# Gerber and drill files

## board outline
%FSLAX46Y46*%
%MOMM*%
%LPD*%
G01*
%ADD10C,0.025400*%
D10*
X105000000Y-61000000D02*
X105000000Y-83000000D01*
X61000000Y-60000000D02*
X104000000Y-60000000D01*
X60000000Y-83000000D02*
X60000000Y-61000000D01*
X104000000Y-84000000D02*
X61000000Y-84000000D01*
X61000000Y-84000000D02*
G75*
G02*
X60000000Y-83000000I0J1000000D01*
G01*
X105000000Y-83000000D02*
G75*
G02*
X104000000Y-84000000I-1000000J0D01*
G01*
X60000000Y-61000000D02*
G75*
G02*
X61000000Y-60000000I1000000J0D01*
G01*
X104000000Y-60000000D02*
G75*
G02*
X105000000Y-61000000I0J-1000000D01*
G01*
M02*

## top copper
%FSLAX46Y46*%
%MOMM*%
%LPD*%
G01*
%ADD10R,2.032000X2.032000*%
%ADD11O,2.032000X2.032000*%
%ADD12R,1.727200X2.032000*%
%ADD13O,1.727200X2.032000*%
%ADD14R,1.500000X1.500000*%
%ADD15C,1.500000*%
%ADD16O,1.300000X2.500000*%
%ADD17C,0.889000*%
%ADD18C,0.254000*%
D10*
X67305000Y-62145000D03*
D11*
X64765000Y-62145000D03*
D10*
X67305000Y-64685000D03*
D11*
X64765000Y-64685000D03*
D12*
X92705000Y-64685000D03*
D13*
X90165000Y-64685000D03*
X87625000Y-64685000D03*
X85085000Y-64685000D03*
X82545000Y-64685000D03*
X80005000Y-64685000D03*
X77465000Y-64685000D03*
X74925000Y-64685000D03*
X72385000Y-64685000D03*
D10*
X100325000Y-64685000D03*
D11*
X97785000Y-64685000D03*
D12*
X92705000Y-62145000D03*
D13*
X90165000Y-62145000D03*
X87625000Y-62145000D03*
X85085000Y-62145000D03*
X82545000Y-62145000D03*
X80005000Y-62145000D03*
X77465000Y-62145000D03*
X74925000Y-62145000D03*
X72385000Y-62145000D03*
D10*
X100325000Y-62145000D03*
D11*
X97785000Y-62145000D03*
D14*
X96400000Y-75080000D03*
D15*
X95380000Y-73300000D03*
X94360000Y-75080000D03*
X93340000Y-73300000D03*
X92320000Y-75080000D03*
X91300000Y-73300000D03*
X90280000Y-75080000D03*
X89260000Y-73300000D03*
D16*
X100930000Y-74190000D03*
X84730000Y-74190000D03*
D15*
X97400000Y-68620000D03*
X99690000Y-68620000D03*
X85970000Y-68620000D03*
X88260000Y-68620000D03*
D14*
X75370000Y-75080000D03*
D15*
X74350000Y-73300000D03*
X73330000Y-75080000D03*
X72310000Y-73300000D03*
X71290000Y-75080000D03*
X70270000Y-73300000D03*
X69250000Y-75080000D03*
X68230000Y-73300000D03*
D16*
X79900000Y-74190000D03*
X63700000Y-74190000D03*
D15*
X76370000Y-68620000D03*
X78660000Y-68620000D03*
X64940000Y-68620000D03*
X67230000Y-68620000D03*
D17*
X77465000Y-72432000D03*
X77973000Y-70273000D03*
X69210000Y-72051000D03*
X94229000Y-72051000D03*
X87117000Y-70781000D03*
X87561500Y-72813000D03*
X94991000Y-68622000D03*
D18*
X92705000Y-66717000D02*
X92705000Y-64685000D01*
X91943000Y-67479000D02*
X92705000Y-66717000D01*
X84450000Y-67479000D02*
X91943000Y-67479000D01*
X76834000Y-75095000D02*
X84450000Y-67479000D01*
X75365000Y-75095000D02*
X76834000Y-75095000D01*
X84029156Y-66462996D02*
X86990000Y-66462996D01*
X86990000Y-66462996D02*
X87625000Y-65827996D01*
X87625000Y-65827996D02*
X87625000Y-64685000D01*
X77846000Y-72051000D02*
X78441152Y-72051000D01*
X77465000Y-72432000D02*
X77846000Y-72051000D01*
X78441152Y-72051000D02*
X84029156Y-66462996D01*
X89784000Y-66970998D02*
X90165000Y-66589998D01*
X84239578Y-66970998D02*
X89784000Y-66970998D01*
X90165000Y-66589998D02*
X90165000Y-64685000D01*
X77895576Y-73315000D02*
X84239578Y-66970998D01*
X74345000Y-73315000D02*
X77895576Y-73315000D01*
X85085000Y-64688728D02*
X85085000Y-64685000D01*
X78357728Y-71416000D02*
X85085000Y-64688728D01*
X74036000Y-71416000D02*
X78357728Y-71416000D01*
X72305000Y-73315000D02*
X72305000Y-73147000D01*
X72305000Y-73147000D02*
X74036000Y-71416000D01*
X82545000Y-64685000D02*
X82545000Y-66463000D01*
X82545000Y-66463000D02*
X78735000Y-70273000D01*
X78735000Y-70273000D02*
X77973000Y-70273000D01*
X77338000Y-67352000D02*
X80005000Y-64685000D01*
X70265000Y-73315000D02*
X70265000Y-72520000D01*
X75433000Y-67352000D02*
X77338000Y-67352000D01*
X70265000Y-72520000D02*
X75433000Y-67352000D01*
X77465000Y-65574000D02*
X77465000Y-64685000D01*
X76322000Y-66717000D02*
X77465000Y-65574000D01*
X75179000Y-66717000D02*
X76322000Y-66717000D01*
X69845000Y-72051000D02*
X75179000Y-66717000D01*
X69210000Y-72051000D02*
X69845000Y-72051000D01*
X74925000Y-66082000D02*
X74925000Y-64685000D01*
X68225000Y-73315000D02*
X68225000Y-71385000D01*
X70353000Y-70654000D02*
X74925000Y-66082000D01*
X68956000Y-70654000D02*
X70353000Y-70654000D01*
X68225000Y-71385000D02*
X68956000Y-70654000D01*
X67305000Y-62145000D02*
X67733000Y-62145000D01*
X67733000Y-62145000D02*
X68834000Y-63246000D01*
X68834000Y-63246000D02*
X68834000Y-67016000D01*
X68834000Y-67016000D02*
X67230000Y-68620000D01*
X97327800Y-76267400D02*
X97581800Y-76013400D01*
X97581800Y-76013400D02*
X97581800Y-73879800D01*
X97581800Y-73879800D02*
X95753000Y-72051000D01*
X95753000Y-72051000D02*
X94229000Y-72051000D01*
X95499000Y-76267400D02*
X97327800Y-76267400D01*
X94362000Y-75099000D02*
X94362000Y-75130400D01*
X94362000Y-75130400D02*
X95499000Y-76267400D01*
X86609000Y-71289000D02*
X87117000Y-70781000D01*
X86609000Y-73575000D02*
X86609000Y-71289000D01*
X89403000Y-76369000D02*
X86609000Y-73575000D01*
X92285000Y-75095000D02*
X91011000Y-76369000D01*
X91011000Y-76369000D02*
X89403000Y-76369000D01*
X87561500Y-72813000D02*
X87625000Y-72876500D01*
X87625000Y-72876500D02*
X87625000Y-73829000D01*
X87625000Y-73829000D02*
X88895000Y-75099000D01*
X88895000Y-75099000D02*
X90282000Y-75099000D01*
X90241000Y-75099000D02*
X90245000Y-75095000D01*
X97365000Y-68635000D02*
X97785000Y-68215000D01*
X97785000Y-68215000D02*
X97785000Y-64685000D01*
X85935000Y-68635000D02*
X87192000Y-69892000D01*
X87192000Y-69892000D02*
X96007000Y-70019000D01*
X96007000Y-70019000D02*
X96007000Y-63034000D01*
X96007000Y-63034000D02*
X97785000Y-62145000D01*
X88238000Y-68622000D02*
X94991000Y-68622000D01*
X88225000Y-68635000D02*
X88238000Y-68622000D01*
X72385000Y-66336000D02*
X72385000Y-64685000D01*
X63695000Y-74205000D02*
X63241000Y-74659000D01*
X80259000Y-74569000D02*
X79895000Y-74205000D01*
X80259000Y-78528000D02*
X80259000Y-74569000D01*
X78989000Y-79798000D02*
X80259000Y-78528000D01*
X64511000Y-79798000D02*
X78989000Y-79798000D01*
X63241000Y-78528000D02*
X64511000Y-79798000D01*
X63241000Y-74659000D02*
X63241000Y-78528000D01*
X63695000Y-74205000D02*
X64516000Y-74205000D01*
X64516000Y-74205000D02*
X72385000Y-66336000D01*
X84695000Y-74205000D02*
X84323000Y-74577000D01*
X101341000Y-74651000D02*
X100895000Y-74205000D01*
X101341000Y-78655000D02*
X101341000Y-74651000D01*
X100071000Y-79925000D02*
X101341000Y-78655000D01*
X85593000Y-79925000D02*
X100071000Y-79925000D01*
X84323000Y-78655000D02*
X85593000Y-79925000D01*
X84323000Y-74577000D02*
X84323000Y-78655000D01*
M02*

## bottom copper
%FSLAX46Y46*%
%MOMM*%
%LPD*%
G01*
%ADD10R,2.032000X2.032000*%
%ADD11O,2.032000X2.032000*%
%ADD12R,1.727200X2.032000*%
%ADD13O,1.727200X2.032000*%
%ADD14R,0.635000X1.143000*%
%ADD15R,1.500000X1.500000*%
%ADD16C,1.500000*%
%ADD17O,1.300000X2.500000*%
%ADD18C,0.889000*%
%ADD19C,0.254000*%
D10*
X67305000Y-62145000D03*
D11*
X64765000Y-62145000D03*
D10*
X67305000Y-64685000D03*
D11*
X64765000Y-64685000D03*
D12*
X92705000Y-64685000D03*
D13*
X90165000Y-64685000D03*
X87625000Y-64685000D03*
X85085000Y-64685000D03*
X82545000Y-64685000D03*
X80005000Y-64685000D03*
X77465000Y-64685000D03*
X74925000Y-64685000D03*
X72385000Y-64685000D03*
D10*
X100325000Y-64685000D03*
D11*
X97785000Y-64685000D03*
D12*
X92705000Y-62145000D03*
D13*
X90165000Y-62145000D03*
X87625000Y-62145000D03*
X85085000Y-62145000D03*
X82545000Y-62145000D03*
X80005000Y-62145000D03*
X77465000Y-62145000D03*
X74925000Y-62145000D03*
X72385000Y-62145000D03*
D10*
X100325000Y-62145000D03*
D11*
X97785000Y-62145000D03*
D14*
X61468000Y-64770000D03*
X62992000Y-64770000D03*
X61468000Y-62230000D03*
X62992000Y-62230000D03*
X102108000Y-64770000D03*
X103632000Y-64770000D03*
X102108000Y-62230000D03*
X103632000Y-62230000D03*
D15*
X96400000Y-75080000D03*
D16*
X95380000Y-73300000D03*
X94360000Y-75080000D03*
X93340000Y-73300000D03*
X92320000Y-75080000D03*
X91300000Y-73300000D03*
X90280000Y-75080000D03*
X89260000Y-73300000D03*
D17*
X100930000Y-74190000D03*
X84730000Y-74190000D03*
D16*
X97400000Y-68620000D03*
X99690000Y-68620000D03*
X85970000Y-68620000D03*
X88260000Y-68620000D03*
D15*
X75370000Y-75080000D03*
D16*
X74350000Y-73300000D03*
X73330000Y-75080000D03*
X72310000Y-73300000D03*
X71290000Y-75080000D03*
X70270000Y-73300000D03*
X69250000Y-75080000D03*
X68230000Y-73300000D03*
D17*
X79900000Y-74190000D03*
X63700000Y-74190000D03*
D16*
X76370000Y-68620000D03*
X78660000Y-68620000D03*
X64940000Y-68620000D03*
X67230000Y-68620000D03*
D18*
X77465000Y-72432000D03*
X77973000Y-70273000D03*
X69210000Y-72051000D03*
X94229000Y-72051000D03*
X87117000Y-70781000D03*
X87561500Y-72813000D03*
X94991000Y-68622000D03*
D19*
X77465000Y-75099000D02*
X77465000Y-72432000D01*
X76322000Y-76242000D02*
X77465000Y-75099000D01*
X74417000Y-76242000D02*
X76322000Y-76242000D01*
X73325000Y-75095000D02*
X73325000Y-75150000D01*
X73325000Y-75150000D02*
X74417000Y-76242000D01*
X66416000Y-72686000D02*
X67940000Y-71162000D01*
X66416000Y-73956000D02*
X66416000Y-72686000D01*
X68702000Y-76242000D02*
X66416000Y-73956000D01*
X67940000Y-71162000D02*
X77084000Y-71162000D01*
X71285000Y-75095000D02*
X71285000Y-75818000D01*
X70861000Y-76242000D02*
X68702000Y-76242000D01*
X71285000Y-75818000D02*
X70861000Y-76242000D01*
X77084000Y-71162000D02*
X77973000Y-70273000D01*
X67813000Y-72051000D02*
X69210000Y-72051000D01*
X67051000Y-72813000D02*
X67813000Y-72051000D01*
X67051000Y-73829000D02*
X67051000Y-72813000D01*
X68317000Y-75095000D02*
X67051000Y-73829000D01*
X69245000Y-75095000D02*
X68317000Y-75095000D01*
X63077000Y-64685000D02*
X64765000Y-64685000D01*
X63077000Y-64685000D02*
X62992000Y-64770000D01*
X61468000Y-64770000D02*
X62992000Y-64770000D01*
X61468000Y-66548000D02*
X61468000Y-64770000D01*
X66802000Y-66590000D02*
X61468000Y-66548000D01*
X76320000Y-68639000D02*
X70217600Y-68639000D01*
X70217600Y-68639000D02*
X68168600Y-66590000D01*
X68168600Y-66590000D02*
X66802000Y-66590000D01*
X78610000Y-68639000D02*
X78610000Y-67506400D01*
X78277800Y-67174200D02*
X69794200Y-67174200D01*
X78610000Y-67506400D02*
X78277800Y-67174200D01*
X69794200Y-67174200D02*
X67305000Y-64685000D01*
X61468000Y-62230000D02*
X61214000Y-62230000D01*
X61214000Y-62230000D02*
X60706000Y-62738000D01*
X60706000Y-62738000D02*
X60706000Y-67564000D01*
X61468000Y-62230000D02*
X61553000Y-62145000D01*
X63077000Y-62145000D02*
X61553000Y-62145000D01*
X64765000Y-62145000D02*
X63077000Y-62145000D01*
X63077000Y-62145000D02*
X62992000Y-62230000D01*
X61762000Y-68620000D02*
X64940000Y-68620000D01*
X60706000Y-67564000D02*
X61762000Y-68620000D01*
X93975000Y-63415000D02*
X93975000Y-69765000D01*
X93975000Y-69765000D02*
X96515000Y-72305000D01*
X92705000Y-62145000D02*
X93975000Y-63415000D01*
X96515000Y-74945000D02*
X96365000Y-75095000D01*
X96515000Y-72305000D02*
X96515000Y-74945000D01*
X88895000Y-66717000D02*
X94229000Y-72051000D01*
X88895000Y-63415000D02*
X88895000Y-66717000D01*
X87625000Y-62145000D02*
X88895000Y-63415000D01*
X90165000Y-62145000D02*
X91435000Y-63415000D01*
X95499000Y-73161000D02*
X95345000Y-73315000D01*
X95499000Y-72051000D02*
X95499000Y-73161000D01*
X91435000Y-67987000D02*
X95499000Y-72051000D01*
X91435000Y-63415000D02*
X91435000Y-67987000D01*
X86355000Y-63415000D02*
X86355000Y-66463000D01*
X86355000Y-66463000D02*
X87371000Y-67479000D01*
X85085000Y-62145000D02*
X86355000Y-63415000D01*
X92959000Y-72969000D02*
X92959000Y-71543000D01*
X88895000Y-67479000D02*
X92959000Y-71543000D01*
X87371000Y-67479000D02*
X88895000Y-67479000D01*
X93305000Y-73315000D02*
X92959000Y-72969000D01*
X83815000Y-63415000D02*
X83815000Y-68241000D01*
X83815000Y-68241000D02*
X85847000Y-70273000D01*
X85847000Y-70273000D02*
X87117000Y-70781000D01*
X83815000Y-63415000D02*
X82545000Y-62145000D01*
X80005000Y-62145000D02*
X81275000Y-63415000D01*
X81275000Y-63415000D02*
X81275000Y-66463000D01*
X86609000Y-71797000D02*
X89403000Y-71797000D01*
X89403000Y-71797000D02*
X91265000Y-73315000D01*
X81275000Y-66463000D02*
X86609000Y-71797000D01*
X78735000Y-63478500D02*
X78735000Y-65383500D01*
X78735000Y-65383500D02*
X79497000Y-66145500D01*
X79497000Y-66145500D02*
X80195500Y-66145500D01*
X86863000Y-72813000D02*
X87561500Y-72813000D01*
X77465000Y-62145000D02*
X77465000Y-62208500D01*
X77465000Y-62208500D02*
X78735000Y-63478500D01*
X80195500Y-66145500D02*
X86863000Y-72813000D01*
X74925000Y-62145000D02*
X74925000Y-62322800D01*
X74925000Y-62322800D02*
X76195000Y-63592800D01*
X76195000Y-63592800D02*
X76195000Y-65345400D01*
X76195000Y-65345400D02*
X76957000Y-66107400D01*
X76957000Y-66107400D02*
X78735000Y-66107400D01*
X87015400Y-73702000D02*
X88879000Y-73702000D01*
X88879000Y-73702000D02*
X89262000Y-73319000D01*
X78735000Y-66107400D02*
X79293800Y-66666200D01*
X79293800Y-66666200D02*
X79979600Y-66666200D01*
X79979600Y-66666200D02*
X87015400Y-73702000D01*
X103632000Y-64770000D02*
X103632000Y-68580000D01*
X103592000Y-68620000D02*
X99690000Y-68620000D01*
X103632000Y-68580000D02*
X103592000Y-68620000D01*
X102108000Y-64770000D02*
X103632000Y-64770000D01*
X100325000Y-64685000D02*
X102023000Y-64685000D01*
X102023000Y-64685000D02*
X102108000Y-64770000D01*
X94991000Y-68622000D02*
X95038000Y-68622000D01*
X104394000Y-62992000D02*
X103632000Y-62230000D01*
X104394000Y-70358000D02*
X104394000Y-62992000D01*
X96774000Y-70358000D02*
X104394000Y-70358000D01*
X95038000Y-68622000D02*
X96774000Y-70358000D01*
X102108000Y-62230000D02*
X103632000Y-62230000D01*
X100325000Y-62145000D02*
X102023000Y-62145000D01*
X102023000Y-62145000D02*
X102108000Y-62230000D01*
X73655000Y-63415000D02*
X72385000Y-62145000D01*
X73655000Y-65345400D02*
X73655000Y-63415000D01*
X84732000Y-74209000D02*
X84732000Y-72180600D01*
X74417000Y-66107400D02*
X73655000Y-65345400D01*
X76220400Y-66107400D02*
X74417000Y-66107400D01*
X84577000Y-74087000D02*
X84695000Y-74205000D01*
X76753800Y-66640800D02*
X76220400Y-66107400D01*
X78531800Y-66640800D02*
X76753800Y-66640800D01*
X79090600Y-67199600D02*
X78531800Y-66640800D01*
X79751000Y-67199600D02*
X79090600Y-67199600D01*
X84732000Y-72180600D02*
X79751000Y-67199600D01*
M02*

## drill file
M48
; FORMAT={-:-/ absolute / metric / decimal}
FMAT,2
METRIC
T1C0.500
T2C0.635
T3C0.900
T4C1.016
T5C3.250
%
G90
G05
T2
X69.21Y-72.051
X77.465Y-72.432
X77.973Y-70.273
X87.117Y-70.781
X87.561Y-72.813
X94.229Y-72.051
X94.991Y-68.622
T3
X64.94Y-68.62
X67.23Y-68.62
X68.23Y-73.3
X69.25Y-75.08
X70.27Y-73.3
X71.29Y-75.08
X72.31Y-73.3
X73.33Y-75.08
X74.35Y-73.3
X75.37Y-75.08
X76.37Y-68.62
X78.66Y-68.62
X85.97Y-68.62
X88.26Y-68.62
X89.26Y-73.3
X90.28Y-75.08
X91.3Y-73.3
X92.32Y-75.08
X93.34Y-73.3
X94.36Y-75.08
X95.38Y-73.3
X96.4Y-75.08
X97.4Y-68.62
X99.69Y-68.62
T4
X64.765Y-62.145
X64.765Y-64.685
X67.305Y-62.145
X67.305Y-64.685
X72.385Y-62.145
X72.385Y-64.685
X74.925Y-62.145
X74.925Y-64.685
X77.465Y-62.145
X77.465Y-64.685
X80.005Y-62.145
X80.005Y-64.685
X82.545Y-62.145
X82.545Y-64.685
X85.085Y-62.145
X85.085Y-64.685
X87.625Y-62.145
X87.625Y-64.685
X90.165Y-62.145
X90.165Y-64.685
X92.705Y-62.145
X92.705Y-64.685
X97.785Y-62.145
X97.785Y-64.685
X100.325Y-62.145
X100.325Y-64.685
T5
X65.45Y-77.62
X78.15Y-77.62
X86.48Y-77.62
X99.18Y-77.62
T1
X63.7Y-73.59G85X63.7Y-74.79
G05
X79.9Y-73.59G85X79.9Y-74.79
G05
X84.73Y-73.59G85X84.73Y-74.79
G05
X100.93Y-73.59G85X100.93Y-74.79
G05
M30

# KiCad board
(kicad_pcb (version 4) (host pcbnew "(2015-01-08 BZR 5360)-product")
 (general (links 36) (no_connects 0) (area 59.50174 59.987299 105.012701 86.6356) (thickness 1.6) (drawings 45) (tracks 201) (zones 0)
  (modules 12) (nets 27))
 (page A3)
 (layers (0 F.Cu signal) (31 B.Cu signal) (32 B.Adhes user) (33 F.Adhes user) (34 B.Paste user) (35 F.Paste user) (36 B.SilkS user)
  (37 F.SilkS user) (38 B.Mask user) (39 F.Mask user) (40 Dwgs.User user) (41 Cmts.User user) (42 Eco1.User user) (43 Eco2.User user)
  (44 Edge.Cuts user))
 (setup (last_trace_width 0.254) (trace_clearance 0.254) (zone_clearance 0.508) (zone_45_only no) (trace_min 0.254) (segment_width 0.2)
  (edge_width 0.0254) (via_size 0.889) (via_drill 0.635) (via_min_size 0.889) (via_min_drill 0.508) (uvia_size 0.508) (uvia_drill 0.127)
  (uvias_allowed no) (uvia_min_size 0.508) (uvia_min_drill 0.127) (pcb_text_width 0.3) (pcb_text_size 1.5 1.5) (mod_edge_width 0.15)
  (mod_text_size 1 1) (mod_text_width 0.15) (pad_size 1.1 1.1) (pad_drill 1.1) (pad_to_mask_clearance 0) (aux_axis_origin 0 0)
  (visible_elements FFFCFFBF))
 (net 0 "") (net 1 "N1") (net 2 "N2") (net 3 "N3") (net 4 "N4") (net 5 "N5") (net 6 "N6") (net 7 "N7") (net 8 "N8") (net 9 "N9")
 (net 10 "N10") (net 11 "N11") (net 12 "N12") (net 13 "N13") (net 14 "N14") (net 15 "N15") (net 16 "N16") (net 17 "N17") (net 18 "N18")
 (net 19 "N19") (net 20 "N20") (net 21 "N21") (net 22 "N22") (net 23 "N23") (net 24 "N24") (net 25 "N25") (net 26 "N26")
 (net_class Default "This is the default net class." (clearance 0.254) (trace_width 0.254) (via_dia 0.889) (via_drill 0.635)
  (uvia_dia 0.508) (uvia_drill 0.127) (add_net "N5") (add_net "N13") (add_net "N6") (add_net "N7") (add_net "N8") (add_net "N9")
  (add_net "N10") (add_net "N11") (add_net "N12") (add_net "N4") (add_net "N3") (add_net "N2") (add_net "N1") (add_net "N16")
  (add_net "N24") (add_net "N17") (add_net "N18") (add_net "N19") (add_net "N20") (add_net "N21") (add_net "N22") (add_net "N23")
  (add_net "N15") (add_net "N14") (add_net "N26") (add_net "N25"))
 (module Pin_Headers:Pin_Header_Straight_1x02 (layer F.Cu) (at 66.035 62.145 180)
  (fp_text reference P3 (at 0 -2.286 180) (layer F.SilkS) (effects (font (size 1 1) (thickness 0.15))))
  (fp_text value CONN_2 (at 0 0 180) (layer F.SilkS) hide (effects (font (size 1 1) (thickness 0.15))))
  (pad 1 thru_hole rect (at -1.27 0 180) (size 2.032 2.032) (drill 1.016) (layers *.Cu *.Mask F.SilkS) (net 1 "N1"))
  (pad 2 thru_hole oval (at 1.27 0 180) (size 2.032 2.032) (drill 1.016) (layers *.Cu *.Mask F.SilkS) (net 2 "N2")))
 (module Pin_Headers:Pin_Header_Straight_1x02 (layer F.Cu) (at 66.035 64.685 180)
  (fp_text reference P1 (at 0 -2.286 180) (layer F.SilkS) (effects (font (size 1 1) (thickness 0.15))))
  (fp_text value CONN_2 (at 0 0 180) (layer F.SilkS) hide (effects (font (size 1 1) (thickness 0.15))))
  (pad 1 thru_hole rect (at -1.27 0 180) (size 2.032 2.032) (drill 1.016) (layers *.Cu *.Mask F.SilkS) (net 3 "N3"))
  (pad 2 thru_hole oval (at 1.27 0 180) (size 2.032 2.032) (drill 1.016) (layers *.Cu *.Mask F.SilkS) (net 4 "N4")))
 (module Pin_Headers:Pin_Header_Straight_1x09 (layer F.Cu) (at 82.545 64.685 180)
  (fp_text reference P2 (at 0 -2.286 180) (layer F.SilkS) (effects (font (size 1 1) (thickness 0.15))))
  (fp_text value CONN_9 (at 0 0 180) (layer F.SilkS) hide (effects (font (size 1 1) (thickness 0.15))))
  (pad 1 thru_hole rect (at -10.16 0 180) (size 1.7272 2.032) (drill 1.016) (layers *.Cu *.Mask F.SilkS) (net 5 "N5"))
  (pad 2 thru_hole oval (at -7.62 0 180) (size 1.7272 2.032) (drill 1.016) (layers *.Cu *.Mask F.SilkS) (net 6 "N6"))
  (pad 3 thru_hole oval (at -5.08 0 180) (size 1.7272 2.032) (drill 1.016) (layers *.Cu *.Mask F.SilkS) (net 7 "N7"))
  (pad 4 thru_hole oval (at -2.54 0 180) (size 1.7272 2.032) (drill 1.016) (layers *.Cu *.Mask F.SilkS) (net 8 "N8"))
  (pad 5 thru_hole oval (at 0 0 180) (size 1.7272 2.032) (drill 1.016) (layers *.Cu *.Mask F.SilkS) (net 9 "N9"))
  (pad 6 thru_hole oval (at 2.54 0 180) (size 1.7272 2.032) (drill 1.016) (layers *.Cu *.Mask F.SilkS) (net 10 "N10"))
  (pad 7 thru_hole oval (at 5.08 0 180) (size 1.7272 2.032) (drill 1.016) (layers *.Cu *.Mask F.SilkS) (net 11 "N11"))
  (pad 8 thru_hole oval (at 7.62 0 180) (size 1.7272 2.032) (drill 1.016) (layers *.Cu *.Mask F.SilkS) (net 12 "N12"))
  (pad 9 thru_hole oval (at 10.16 0 180) (size 1.7272 2.032) (drill 1.016) (layers *.Cu *.Mask F.SilkS) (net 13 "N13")))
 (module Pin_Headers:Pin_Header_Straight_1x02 (layer F.Cu) (at 99.055 64.685 180)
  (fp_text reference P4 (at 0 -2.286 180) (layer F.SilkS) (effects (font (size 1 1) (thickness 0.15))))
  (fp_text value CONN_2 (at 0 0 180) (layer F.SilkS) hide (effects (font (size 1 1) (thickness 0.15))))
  (pad 1 thru_hole rect (at -1.27 0 180) (size 2.032 2.032) (drill 1.016) (layers *.Cu *.Mask F.SilkS) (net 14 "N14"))
  (pad 2 thru_hole oval (at 1.27 0 180) (size 2.032 2.032) (drill 1.016) (layers *.Cu *.Mask F.SilkS) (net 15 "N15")))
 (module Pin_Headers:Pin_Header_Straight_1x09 (layer F.Cu) (at 82.545 62.145 180)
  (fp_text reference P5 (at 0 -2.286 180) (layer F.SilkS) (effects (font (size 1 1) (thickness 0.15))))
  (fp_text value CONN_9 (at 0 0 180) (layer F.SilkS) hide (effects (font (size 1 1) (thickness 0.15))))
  (pad 1 thru_hole rect (at -10.16 0 180) (size 1.7272 2.032) (drill 1.016) (layers *.Cu *.Mask F.SilkS) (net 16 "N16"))
  (pad 2 thru_hole oval (at -7.62 0 180) (size 1.7272 2.032) (drill 1.016) (layers *.Cu *.Mask F.SilkS) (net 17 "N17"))
  (pad 3 thru_hole oval (at -5.08 0 180) (size 1.7272 2.032) (drill 1.016) (layers *.Cu *.Mask F.SilkS) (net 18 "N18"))
  (pad 4 thru_hole oval (at -2.54 0 180) (size 1.7272 2.032) (drill 1.016) (layers *.Cu *.Mask F.SilkS) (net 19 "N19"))
  (pad 5 thru_hole oval (at 0 0 180) (size 1.7272 2.032) (drill 1.016) (layers *.Cu *.Mask F.SilkS) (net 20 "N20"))
  (pad 6 thru_hole oval (at 2.54 0 180) (size 1.7272 2.032) (drill 1.016) (layers *.Cu *.Mask F.SilkS) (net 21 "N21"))
  (pad 7 thru_hole oval (at 5.08 0 180) (size 1.7272 2.032) (drill 1.016) (layers *.Cu *.Mask F.SilkS) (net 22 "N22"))
  (pad 8 thru_hole oval (at 7.62 0 180) (size 1.7272 2.032) (drill 1.016) (layers *.Cu *.Mask F.SilkS) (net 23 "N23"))
  (pad 9 thru_hole oval (at 10.16 0 180) (size 1.7272 2.032) (drill 1.016) (layers *.Cu *.Mask F.SilkS) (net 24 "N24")))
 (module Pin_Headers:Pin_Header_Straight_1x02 (layer F.Cu) (at 99.055 62.145 180)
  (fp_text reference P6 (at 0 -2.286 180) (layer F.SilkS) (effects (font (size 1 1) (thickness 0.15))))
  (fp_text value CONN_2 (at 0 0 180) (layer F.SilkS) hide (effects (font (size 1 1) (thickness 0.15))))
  (pad 1 thru_hole rect (at -1.27 0 180) (size 2.032 2.032) (drill 1.016) (layers *.Cu *.Mask F.SilkS) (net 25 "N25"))
  (pad 2 thru_hole oval (at 1.27 0 180) (size 2.032 2.032) (drill 1.016) (layers *.Cu *.Mask F.SilkS) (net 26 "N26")))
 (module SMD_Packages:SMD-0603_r (layer B.Cu) (at 62.23 64.77)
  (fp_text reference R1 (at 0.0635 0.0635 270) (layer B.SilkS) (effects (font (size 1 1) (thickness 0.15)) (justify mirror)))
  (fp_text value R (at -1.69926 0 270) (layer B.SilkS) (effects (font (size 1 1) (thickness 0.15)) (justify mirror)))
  (pad 1 smd rect (at -0.762 0) (size 0.635 1.143) (layers B.Cu B.Paste B.Mask) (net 4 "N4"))
  (pad 2 smd rect (at 0.762 0) (size 0.635 1.143) (layers B.Cu B.Paste B.Mask) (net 4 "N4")))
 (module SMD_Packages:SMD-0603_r (layer B.Cu) (at 62.23 62.23)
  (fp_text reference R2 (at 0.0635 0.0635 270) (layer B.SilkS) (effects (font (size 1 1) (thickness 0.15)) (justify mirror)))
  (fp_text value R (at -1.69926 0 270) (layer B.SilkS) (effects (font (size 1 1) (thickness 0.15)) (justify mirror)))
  (pad 1 smd rect (at -0.762 0) (size 0.635 1.143) (layers B.Cu B.Paste B.Mask) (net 2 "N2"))
  (pad 2 smd rect (at 0.762 0) (size 0.635 1.143) (layers B.Cu B.Paste B.Mask) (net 2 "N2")))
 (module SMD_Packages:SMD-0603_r (layer B.Cu) (at 102.87 64.77)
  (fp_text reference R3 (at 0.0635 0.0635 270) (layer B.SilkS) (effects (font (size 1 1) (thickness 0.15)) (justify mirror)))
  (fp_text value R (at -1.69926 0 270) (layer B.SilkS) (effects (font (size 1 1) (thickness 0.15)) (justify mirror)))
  (pad 1 smd rect (at -0.762 0) (size 0.635 1.143) (layers B.Cu B.Paste B.Mask) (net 14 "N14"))
  (pad 2 smd rect (at 0.762 0) (size 0.635 1.143) (layers B.Cu B.Paste B.Mask) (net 14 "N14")))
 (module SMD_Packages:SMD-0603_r (layer B.Cu) (at 102.87 62.23)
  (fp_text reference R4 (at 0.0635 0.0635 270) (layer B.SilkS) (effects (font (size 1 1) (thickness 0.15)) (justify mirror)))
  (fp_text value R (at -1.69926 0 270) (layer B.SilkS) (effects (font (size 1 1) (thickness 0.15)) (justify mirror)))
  (pad 1 smd rect (at -0.762 0) (size 0.635 1.143) (layers B.Cu B.Paste B.Mask) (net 25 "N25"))
  (pad 2 smd rect (at 0.762 0) (size 0.635 1.143) (layers B.Cu B.Paste B.Mask) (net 25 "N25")))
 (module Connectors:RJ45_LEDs (layer F.Cu) (at 96.4 75.08 180)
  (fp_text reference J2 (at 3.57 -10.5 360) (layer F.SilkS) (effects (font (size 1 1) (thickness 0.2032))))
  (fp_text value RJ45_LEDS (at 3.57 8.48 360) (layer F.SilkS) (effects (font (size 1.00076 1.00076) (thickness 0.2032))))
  (pad 1 thru_hole rect (at 0 0) (size 1.5 1.5) (drill 0.9) (layers *.Cu *.Mask F.SilkS) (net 16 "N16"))
  (pad 2 thru_hole circle (at 1.02 1.78) (size 1.5 1.5) (drill 0.9) (layers *.Cu *.Mask F.SilkS) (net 17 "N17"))
  (pad 3 thru_hole circle (at 2.04 0) (size 1.5 1.5) (drill 0.9) (layers *.Cu *.Mask F.SilkS) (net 18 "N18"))
  (pad 4 thru_hole circle (at 3.06 1.78) (size 1.5 1.5) (drill 0.9) (layers *.Cu *.Mask F.SilkS) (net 19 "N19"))
  (pad 5 thru_hole circle (at 4.08 0) (size 1.5 1.5) (drill 0.9) (layers *.Cu *.Mask F.SilkS) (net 20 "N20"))
  (pad 6 thru_hole circle (at 5.1 1.78) (size 1.5 1.5) (drill 0.9) (layers *.Cu *.Mask F.SilkS) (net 21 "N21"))
  (pad 7 thru_hole circle (at 6.12 0) (size 1.5 1.5) (drill 0.9) (layers *.Cu *.Mask F.SilkS) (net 22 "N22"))
  (pad 8 thru_hole circle (at 7.14 1.78) (size 1.5 1.5) (drill 0.9) (layers *.Cu *.Mask F.SilkS) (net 23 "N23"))
  (pad 13 thru_hole oval (at -4.53 0.89) (size 1.3 2.5) (drill oval 0.5 1.7) (layers *.Cu *.Mask F.SilkS) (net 24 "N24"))
  (pad 13 thru_hole oval (at 11.67 0.89) (size 1.3 2.5) (drill oval 0.5 1.7) (layers *.Cu *.Mask F.SilkS) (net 24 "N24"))
  (pad GA thru_hole circle (at -1 6.46) (size 1.5 1.5) (drill 0.9) (layers *.Cu *.Mask F.SilkS) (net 15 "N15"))
  (pad "" np_thru_hole circle (at -2.78 -2.54) (size 3.25 3.25) (drill 3.25) (layers *.Cu *.Mask F.SilkS))
  (pad "" np_thru_hole circle (at 9.92 -2.54) (size 3.25 3.25) (drill 3.25) (layers *.Cu *.Mask F.SilkS))
  (pad GK thru_hole circle (at -3.29 6.46) (size 1.5 1.5) (drill 0.9) (layers *.Cu *.Mask F.SilkS) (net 14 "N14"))
  (pad YA thru_hole circle (at 10.43 6.46) (size 1.5 1.5) (drill 0.9) (layers *.Cu *.Mask F.SilkS) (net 26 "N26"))
  (pad YK thru_hole circle (at 8.14 6.46) (size 1.5 1.5) (drill 0.9) (layers *.Cu *.Mask F.SilkS) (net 25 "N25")))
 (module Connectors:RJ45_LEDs (layer F.Cu) (at 75.37 75.08 180)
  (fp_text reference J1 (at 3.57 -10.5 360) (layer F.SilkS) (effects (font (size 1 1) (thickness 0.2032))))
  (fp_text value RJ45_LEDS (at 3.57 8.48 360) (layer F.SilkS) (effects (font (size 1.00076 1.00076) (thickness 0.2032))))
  (pad 1 thru_hole rect (at 0 0) (size 1.5 1.5) (drill 0.9) (layers *.Cu *.Mask F.SilkS) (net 5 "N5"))
  (pad 2 thru_hole circle (at 1.02 1.78) (size 1.5 1.5) (drill 0.9) (layers *.Cu *.Mask F.SilkS) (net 6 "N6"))
  (pad 3 thru_hole circle (at 2.04 0) (size 1.5 1.5) (drill 0.9) (layers *.Cu *.Mask F.SilkS) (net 7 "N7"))
  (pad 4 thru_hole circle (at 3.06 1.78) (size 1.5 1.5) (drill 0.9) (layers *.Cu *.Mask F.SilkS) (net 8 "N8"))
  (pad 5 thru_hole circle (at 4.08 0) (size 1.5 1.5) (drill 0.9) (layers *.Cu *.Mask F.SilkS) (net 9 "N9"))
  (pad 6 thru_hole circle (at 5.1 1.78) (size 1.5 1.5) (drill 0.9) (layers *.Cu *.Mask F.SilkS) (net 10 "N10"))
  (pad 7 thru_hole circle (at 6.12 0) (size 1.5 1.5) (drill 0.9) (layers *.Cu *.Mask F.SilkS) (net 11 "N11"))
  (pad 8 thru_hole circle (at 7.14 1.78) (size 1.5 1.5) (drill 0.9) (layers *.Cu *.Mask F.SilkS) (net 12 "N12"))
  (pad 13 thru_hole oval (at -4.53 0.89) (size 1.3 2.5) (drill oval 0.5 1.7) (layers *.Cu *.Mask F.SilkS) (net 13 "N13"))
  (pad 13 thru_hole oval (at 11.67 0.89) (size 1.3 2.5) (drill oval 0.5 1.7) (layers *.Cu *.Mask F.SilkS) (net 13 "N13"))
  (pad GA thru_hole circle (at -1 6.46) (size 1.5 1.5) (drill 0.9) (layers *.Cu *.Mask F.SilkS) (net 4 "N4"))
  (pad "" np_thru_hole circle (at -2.78 -2.54) (size 3.25 3.25) (drill 3.25) (layers *.Cu *.Mask F.SilkS))
  (pad "" np_thru_hole circle (at 9.92 -2.54) (size 3.25 3.25) (drill 3.25) (layers *.Cu *.Mask F.SilkS))
  (pad GK thru_hole circle (at -3.29 6.46) (size 1.5 1.5) (drill 0.9) (layers *.Cu *.Mask F.SilkS) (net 3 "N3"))
  (pad YA thru_hole circle (at 10.43 6.46) (size 1.5 1.5) (drill 0.9) (layers *.Cu *.Mask F.SilkS) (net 2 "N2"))
  (pad YK thru_hole circle (at 8.14 6.46) (size 1.5 1.5) (drill 0.9) (layers *.Cu *.Mask F.SilkS) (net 1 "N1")))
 (gr_line (start 105 61) (end 105 83) (angle 90) (layer Edge.Cuts) (width 0.0254))
 (gr_line (start 61 60) (end 104 60) (angle 90) (layer Edge.Cuts) (width 0.0254))
 (gr_line (start 60 83) (end 60 61) (angle 90) (layer Edge.Cuts) (width 0.0254))
 (gr_line (start 104 84) (end 61 84) (angle 90) (layer Edge.Cuts) (width 0.0254))
 (gr_arc (start 61 83) (end 61 84) (angle 90) (layer Edge.Cuts) (width 0.0254))
 (gr_arc (start 104 83) (end 105 83) (angle 90) (layer Edge.Cuts) (width 0.0254))
 (gr_arc (start 61 61) (end 60 61) (angle 90) (layer Edge.Cuts) (width 0.0254))
 (gr_arc (start 104 61) (end 104 60) (angle 90) (layer Edge.Cuts) (width 0.0254))
 (segment (start 92.705 66.717) (end 92.705 64.685) (width 0.254) (layer F.Cu) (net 5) (status 20))
 (segment (start 91.943 67.479) (end 92.705 66.717) (width 0.254) (layer F.Cu) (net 5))
 (segment (start 84.45 67.479) (end 91.943 67.479) (width 0.254) (layer F.Cu) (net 5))
 (segment (start 76.834 75.095) (end 84.45 67.479) (width 0.254) (layer F.Cu) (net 5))
 (segment (start 75.365 75.095) (end 76.834 75.095) (width 0.254) (layer F.Cu) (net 5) (status 10))
 (segment (start 84.029156 66.462996) (end 86.99 66.462996) (width 0.254) (layer F.Cu) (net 7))
 (segment (start 86.99 66.462996) (end 87.625 65.827996) (width 0.254) (layer F.Cu) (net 7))
 (segment (start 87.625 65.827996) (end 87.625 64.685) (width 0.254) (layer F.Cu) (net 7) (status 20))
 (via (at 77.465 72.432) (size 0.889) (layers F.Cu B.Cu) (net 7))
 (segment (start 77.465 75.099) (end 77.465 72.432) (width 0.254) (layer B.Cu) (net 7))
 (segment (start 76.322 76.242) (end 77.465 75.099) (width 0.254) (layer B.Cu) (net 7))
 (segment (start 77.846 72.051) (end 78.441152 72.051) (width 0.254) (layer F.Cu) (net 7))
 (segment (start 77.465 72.432) (end 77.846 72.051) (width 0.254) (layer F.Cu) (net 7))
 (segment (start 78.441152 72.051) (end 84.029156 66.462996) (width 0.254) (layer F.Cu) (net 7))
 (segment (start 74.417 76.242) (end 76.322 76.242) (width 0.254) (layer B.Cu) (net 7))
 (segment (start 73.325 75.095) (end 73.325 75.15) (width 0.254) (layer B.Cu) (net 7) (status 30))
 (segment (start 73.325 75.15) (end 74.417 76.242) (width 0.254) (layer B.Cu) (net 7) (status 10))
 (segment (start 89.784 66.970998) (end 90.165 66.589998) (width 0.254) (layer F.Cu) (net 6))
 (segment (start 84.239578 66.970998) (end 89.784 66.970998) (width 0.254) (layer F.Cu) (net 6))
 (segment (start 90.165 66.589998) (end 90.165 64.685) (width 0.254) (layer F.Cu) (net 6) (status 20))
 (segment (start 77.895576 73.315) (end 84.239578 66.970998) (width 0.254) (layer F.Cu) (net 6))
 (segment (start 74.345 73.315) (end 77.895576 73.315) (width 0.254) (layer F.Cu) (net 6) (status 10))
 (segment (start 85.085 64.688728) (end 85.085 64.685) (width 0.254) (layer F.Cu) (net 8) (status 30))
 (segment (start 78.357728 71.416) (end 85.085 64.688728) (width 0.254) (layer F.Cu) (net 8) (status 20))
 (segment (start 74.036 71.416) (end 78.357728 71.416) (width 0.254) (layer F.Cu) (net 8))
 (segment (start 72.305 73.315) (end 72.305 73.147) (width 0.254) (layer F.Cu) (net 8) (status 30))
 (segment (start 72.305 73.147) (end 74.036 71.416) (width 0.254) (layer F.Cu) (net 8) (status 10))
 (segment (start 82.545 64.685) (end 82.545 66.463) (width 0.254) (layer F.Cu) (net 9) (status 10))
 (segment (start 66.416 72.686) (end 67.94 71.162) (width 0.254) (layer B.Cu) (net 9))
 (segment (start 66.416 73.956) (end 66.416 72.686) (width 0.254) (layer B.Cu) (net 9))
 (segment (start 68.702 76.242) (end 66.416 73.956) (width 0.254) (layer B.Cu) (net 9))
 (segment (start 67.94 71.162) (end 77.084 71.162) (width 0.254) (layer B.Cu) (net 9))
 (segment (start 71.285 75.095) (end 71.285 75.818) (width 0.254) (layer B.Cu) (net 9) (status 30))
 (segment (start 70.861 76.242) (end 68.702 76.242) (width 0.254) (layer B.Cu) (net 9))
 (segment (start 71.285 75.818) (end 70.861 76.242) (width 0.254) (layer B.Cu) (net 9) (status 10))
 (segment (start 77.084 71.162) (end 77.973 70.273) (width 0.254) (layer B.Cu) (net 9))
 (via (at 77.973 70.273) (size 0.889) (layers F.Cu B.Cu) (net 9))
 (segment (start 82.545 66.463) (end 78.735 70.273) (width 0.254) (layer F.Cu) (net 9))
 (segment (start 78.735 70.273) (end 77.973 70.273) (width 0.254) (layer F.Cu) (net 9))
 (segment (start 77.338 67.352) (end 80.005 64.685) (width 0.254) (layer F.Cu) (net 10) (status 20))
 (segment (start 70.265 73.315) (end 70.265 72.52) (width 0.254) (layer F.Cu) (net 10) (status 10))
 (segment (start 75.433 67.352) (end 77.338 67.352) (width 0.254) (layer F.Cu) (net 10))
 (segment (start 70.265 72.52) (end 75.433 67.352) (width 0.254) (layer F.Cu) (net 10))
 (segment (start 77.465 65.574) (end 77.465 64.685) (width 0.254) (layer F.Cu) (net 11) (status 30))
 (segment (start 76.322 66.717) (end 77.465 65.574) (width 0.254) (layer F.Cu) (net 11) (status 20))
 (segment (start 75.179 66.717) (end 76.322 66.717) (width 0.254) (layer F.Cu) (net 11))
 (segment (start 69.845 72.051) (end 75.179 66.717) (width 0.254) (layer F.Cu) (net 11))
 (segment (start 69.21 72.051) (end 69.845 72.051) (width 0.254) (layer F.Cu) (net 11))
 (via (at 69.21 72.051) (size 0.889) (layers F.Cu B.Cu) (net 11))
 (segment (start 67.813 72.051) (end 69.21 72.051) (width 0.254) (layer B.Cu) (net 11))
 (segment (start 67.051 72.813) (end 67.813 72.051) (width 0.254) (layer B.Cu) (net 11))
 (segment (start 67.051 73.829) (end 67.051 72.813) (width 0.254) (layer B.Cu) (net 11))
 (segment (start 68.317 75.095) (end 67.051 73.829) (width 0.254) (layer B.Cu) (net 11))
 (segment (start 69.245 75.095) (end 68.317 75.095) (width 0.254) (layer B.Cu) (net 11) (status 10))
 (segment (start 74.925 66.082) (end 74.925 64.685) (width 0.254) (layer F.Cu) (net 12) (status 20))
 (segment (start 68.225 73.315) (end 68.225 71.385) (width 0.254) (layer F.Cu) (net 12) (status 10))
 (segment (start 70.353 70.654) (end 74.925 66.082) (width 0.254) (layer F.Cu) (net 12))
 (segment (start 68.956 70.654) (end 70.353 70.654) (width 0.254) (layer F.Cu) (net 12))
 (segment (start 68.225 71.385) (end 68.956 70.654) (width 0.254) (layer F.Cu) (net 12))
 (segment (start 63.077 64.685) (end 64.765 64.685) (width 0.254) (layer B.Cu) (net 4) (status 30))
 (segment (start 63.077 64.685) (end 62.992 64.77) (width 0.254) (layer B.Cu) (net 4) (status 30))
 (segment (start 61.468 64.77) (end 62.992 64.77) (width 0.254) (layer B.Cu) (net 4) (status 30))
 (segment (start 61.468 66.548) (end 61.468 64.77) (width 0.254) (layer B.Cu) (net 4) (status 20))
 (segment (start 66.802 66.59) (end 61.468 66.548) (width 0.254) (layer B.Cu) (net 4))
 (segment (start 76.32 68.639) (end 70.2176 68.639) (width 0.254) (layer B.Cu) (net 4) (status 10))
 (segment (start 70.2176 68.639) (end 68.1686 66.59) (width 0.254) (layer B.Cu) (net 4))
 (segment (start 68.1686 66.59) (end 66.802 66.59) (width 0.254) (layer B.Cu) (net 4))
 (segment (start 78.61 68.639) (end 78.61 67.5064) (width 0.254) (layer B.Cu) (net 3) (status 10))
 (segment (start 78.2778 67.1742) (end 69.7942 67.1742) (width 0.254) (layer B.Cu) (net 3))
 (segment (start 78.61 67.5064) (end 78.2778 67.1742) (width 0.254) (layer B.Cu) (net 3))
 (segment (start 69.7942 67.1742) (end 67.305 64.685) (width 0.254) (layer B.Cu) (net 3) (status 20))
 (segment (start 61.468 62.23) (end 61.214 62.23) (width 0.254) (layer B.Cu) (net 2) (status 30))
 (segment (start 61.214 62.23) (end 60.706 62.738) (width 0.254) (layer B.Cu) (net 2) (status 10))
 (segment (start 60.706 62.738) (end 60.706 67.564) (width 0.254) (layer B.Cu) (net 2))
 (segment (start 61.468 62.23) (end 61.553 62.145) (width 0.254) (layer B.Cu) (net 2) (status 30))
 (segment (start 63.077 62.145) (end 61.553 62.145) (width 0.254) (layer B.Cu) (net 2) (status 30))
 (segment (start 64.765 62.145) (end 63.077 62.145) (width 0.254) (layer B.Cu) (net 2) (status 30))
 (segment (start 63.077 62.145) (end 62.992 62.23) (width 0.254) (layer B.Cu) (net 2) (status 30))
 (segment (start 61.762 68.62) (end 64.94 68.62) (width 0.254) (layer B.Cu) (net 2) (status 20))
 (segment (start 60.706 67.564) (end 61.762 68.62) (width 0.254) (layer B.Cu) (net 2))
 (segment (start 67.305 62.145) (end 67.733 62.145) (width 0.254) (layer F.Cu) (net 1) (status 30))
 (segment (start 67.733 62.145) (end 68.834 63.246) (width 0.254) (layer F.Cu) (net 1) (status 10))
 (segment (start 68.834 63.246) (end 68.834 67.016) (width 0.254) (layer F.Cu) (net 1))
 (segment (start 68.834 67.016) (end 67.23 68.62) (width 0.254) (layer F.Cu) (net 1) (status 20))
 (segment (start 93.975 63.415) (end 93.975 69.765) (width 0.254) (layer B.Cu) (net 16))
 (segment (start 93.975 69.765) (end 96.515 72.305) (width 0.254) (layer B.Cu) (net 16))
 (segment (start 92.705 62.145) (end 93.975 63.415) (width 0.254) (layer B.Cu) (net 16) (status 10))
 (segment (start 96.515 74.945) (end 96.365 75.095) (width 0.254) (layer B.Cu) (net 16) (status 30))
 (segment (start 96.515 72.305) (end 96.515 74.945) (width 0.254) (layer B.Cu) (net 16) (status 20))
 (segment (start 97.3278 76.2674) (end 97.5818 76.0134) (width 0.254) (layer F.Cu) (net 18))
 (segment (start 97.5818 76.0134) (end 97.5818 73.8798) (width 0.254) (layer F.Cu) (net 18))
 (segment (start 97.5818 73.8798) (end 95.753 72.051) (width 0.254) (layer F.Cu) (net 18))
 (segment (start 95.753 72.051) (end 94.229 72.051) (width 0.254) (layer F.Cu) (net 18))
 (via (at 94.229 72.051) (size 0.889) (layers F.Cu B.Cu) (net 18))
 (segment (start 88.895 66.717) (end 94.229 72.051) (width 0.254) (layer B.Cu) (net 18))
 (segment (start 88.895 63.415) (end 88.895 66.717) (width 0.254) (layer B.Cu) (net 18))
 (segment (start 87.625 62.145) (end 88.895 63.415) (width 0.254) (layer B.Cu) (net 18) (status 10))
 (segment (start 95.499 76.2674) (end 97.3278 76.2674) (width 0.254) (layer F.Cu) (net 18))
 (segment (start 94.362 75.099) (end 94.362 75.1304) (width 0.254) (layer F.Cu) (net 18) (status 30))
 (segment (start 94.362 75.1304) (end 95.499 76.2674) (width 0.254) (layer F.Cu) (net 18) (status 10))
 (segment (start 90.165 62.145) (end 91.435 63.415) (width 0.254) (layer B.Cu) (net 17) (status 10))
 (segment (start 95.499 73.161) (end 95.345 73.315) (width 0.254) (layer B.Cu) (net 17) (status 30))
 (segment (start 95.499 72.051) (end 95.499 73.161) (width 0.254) (layer B.Cu) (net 17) (status 20))
 (segment (start 91.435 67.987) (end 95.499 72.051) (width 0.254) (layer B.Cu) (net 17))
 (segment (start 91.435 63.415) (end 91.435 67.987) (width 0.254) (layer B.Cu) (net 17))
 (segment (start 86.355 63.415) (end 86.355 66.463) (width 0.254) (layer B.Cu) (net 19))
 (segment (start 86.355 66.463) (end 87.371 67.479) (width 0.254) (layer B.Cu) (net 19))
 (segment (start 85.085 62.145) (end 86.355 63.415) (width 0.254) (layer B.Cu) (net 19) (status 10))
 (segment (start 92.959 72.969) (end 92.959 71.543) (width 0.254) (layer B.Cu) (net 19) (status 10))
 (segment (start 88.895 67.479) (end 92.959 71.543) (width 0.254) (layer B.Cu) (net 19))
 (segment (start 87.371 67.479) (end 88.895 67.479) (width 0.254) (layer B.Cu) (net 19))
 (segment (start 93.305 73.315) (end 92.959 72.969) (width 0.254) (layer B.Cu) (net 19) (status 30))
 (segment (start 83.815 63.415) (end 83.815 68.241) (width 0.254) (layer B.Cu) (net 20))
 (segment (start 83.815 68.241) (end 85.847 70.273) (width 0.254) (layer B.Cu) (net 20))
 (segment (start 85.847 70.273) (end 87.117 70.781) (width 0.254) (layer B.Cu) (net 20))
 (via (at 87.117 70.781) (size 0.889) (layers F.Cu B.Cu) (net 20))
 (segment (start 86.609 71.289) (end 87.117 70.781) (width 0.254) (layer F.Cu) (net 20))
 (segment (start 86.609 73.575) (end 86.609 71.289) (width 0.254) (layer F.Cu) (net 20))
 (segment (start 89.403 76.369) (end 86.609 73.575) (width 0.254) (layer F.Cu) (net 20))
 (segment (start 83.815 63.415) (end 82.545 62.145) (width 0.254) (layer B.Cu) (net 20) (status 20))
 (segment (start 92.285 75.095) (end 91.011 76.369) (width 0.254) (layer F.Cu) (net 20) (status 10))
 (segment (start 91.011 76.369) (end 89.403 76.369) (width 0.254) (layer F.Cu) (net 20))
 (segment (start 80.005 62.145) (end 81.275 63.415) (width 0.254) (layer B.Cu) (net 21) (status 10))
 (segment (start 81.275 63.415) (end 81.275 66.463) (width 0.254) (layer B.Cu) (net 21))
 (segment (start 86.609 71.797) (end 89.403 71.797) (width 0.254) (layer B.Cu) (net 21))
 (segment (start 89.403 71.797) (end 91.265 73.315) (width 0.254) (layer B.Cu) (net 21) (status 20))
 (segment (start 81.275 66.463) (end 86.609 71.797) (width 0.254) (layer B.Cu) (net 21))
 (segment (start 78.735 63.4785) (end 78.735 65.3835) (width 0.254) (layer B.Cu) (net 22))
 (segment (start 78.735 65.3835) (end 79.497 66.1455) (width 0.254) (layer B.Cu) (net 22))
 (segment (start 79.497 66.1455) (end 80.1955 66.1455) (width 0.254) (layer B.Cu) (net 22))
 (segment (start 86.863 72.813) (end 87.5615 72.813) (width 0.254) (layer B.Cu) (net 22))
 (via (at 87.5615 72.813) (size 0.889) (layers F.Cu B.Cu) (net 22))
 (segment (start 87.5615 72.813) (end 87.625 72.8765) (width 0.254) (layer F.Cu) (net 22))
 (segment (start 87.625 72.8765) (end 87.625 73.829) (width 0.254) (layer F.Cu) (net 22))
 (segment (start 87.625 73.829) (end 88.895 75.099) (width 0.254) (layer F.Cu) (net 22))
 (segment (start 77.465 62.145) (end 77.465 62.2085) (width 0.254) (layer B.Cu) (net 22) (status 30))
 (segment (start 77.465 62.2085) (end 78.735 63.4785) (width 0.254) (layer B.Cu) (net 22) (status 10))
 (segment (start 88.895 75.099) (end 90.282 75.099) (width 0.254) (layer F.Cu) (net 22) (status 20))
 (segment (start 90.241 75.099) (end 90.245 75.095) (width 0.254) (layer F.Cu) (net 22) (status 30))
 (segment (start 80.1955 66.1455) (end 86.863 72.813) (width 0.254) (layer B.Cu) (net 22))
 (segment (start 74.925 62.145) (end 74.925 62.3228) (width 0.254) (layer B.Cu) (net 23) (status 30))
 (segment (start 74.925 62.3228) (end 76.195 63.5928) (width 0.254) (layer B.Cu) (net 23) (status 10))
 (segment (start 76.195 63.5928) (end 76.195 65.3454) (width 0.254) (layer B.Cu) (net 23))
 (segment (start 76.195 65.3454) (end 76.957 66.1074) (width 0.254) (layer B.Cu) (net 23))
 (segment (start 76.957 66.1074) (end 78.735 66.1074) (width 0.254) (layer B.Cu) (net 23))
 (segment (start 87.0154 73.702) (end 88.879 73.702) (width 0.254) (layer B.Cu) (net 23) (status 20))
 (segment (start 88.879 73.702) (end 89.262 73.319) (width 0.254) (layer B.Cu) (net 23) (status 30))
 (segment (start 78.735 66.1074) (end 79.2938 66.6662) (width 0.254) (layer B.Cu) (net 23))
 (segment (start 79.2938 66.6662) (end 79.9796 66.6662) (width 0.254) (layer B.Cu) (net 23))
 (segment (start 79.9796 66.6662) (end 87.0154 73.702) (width 0.254) (layer B.Cu) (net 23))
 (segment (start 97.365 68.635) (end 97.785 68.215) (width 0.254) (layer F.Cu) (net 15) (status 30))
 (segment (start 97.785 68.215) (end 97.785 64.685) (width 0.254) (layer F.Cu) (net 15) (status 30))
 (segment (start 103.632 64.77) (end 103.632 68.58) (width 0.254) (layer B.Cu) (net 14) (status 10))
 (segment (start 103.592 68.62) (end 99.69 68.62) (width 0.254) (layer B.Cu) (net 14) (status 20))
 (segment (start 103.632 68.58) (end 103.592 68.62) (width 0.254) (layer B.Cu) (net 14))
 (segment (start 102.108 64.77) (end 103.632 64.77) (width 0.254) (layer B.Cu) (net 14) (status 30))
 (segment (start 100.325 64.685) (end 102.023 64.685) (width 0.254) (layer B.Cu) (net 14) (status 30))
 (segment (start 102.023 64.685) (end 102.108 64.77) (width 0.254) (layer B.Cu) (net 14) (status 30))
 (segment (start 85.935 68.635) (end 87.192 69.892) (width 0.254) (layer F.Cu) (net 26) (status 10))
 (segment (start 87.192 69.892) (end 96.007 70.019) (width 0.254) (layer F.Cu) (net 26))
 (segment (start 96.007 70.019) (end 96.007 63.034) (width 0.254) (layer F.Cu) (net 26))
 (segment (start 96.007 63.034) (end 97.785 62.145) (width 0.254) (layer F.Cu) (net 26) (status 20))
 (segment (start 94.991 68.622) (end 95.038 68.622) (width 0.254) (layer B.Cu) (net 25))
 (via (at 94.991 68.622) (size 0.889) (layers F.Cu B.Cu) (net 25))
 (segment (start 88.238 68.622) (end 94.991 68.622) (width 0.254) (layer F.Cu) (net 25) (status 10))
 (segment (start 104.394 62.992) (end 103.632 62.23) (width 0.254) (layer B.Cu) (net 25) (status 20))
 (segment (start 104.394 70.358) (end 104.394 62.992) (width 0.254) (layer B.Cu) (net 25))
 (segment (start 96.774 70.358) (end 104.394 70.358) (width 0.254) (layer B.Cu) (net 25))
 (segment (start 95.038 68.622) (end 96.774 70.358) (width 0.254) (layer B.Cu) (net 25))
 (segment (start 102.108 62.23) (end 103.632 62.23) (width 0.254) (layer B.Cu) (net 25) (status 30))
 (segment (start 100.325 62.145) (end 102.023 62.145) (width 0.254) (layer B.Cu) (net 25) (status 30))
 (segment (start 102.023 62.145) (end 102.108 62.23) (width 0.254) (layer B.Cu) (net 25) (status 30))
 (segment (start 88.225 68.635) (end 88.238 68.622) (width 0.254) (layer F.Cu) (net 25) (status 30))
 (segment (start 72.385 66.336) (end 72.385 64.685) (width 0.254) (layer F.Cu) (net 13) (status 20))
 (segment (start 63.695 74.205) (end 63.241 74.659) (width 0.254) (layer F.Cu) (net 13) (status 30))
 (segment (start 80.259 74.569) (end 79.895 74.205) (width 0.254) (layer F.Cu) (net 13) (status 30))
 (segment (start 80.259 78.528) (end 80.259 74.569) (width 0.254) (layer F.Cu) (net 13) (status 20))
 (segment (start 78.989 79.798) (end 80.259 78.528) (width 0.254) (layer F.Cu) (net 13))
 (segment (start 64.511 79.798) (end 78.989 79.798) (width 0.254) (layer F.Cu) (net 13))
 (segment (start 63.241 78.528) (end 64.511 79.798) (width 0.254) (layer F.Cu) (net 13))
 (segment (start 63.241 74.659) (end 63.241 78.528) (width 0.254) (layer F.Cu) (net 13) (status 10))
 (segment (start 63.695 74.205) (end 64.516 74.205) (width 0.254) (layer F.Cu) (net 13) (status 10))
 (segment (start 64.516 74.205) (end 72.385 66.336) (width 0.254) (layer F.Cu) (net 13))
 (segment (start 73.655 63.415) (end 72.385 62.145) (width 0.254) (layer B.Cu) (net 24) (status 20))
 (segment (start 73.655 65.3454) (end 73.655 63.415) (width 0.254) (layer B.Cu) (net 24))
 (segment (start 84.732 74.209) (end 84.732 72.1806) (width 0.254) (layer B.Cu) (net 24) (status 10))
 (segment (start 74.417 66.1074) (end 73.655 65.3454) (width 0.254) (layer B.Cu) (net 24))
 (segment (start 76.2204 66.1074) (end 74.417 66.1074) (width 0.254) (layer B.Cu) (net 24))
 (segment (start 84.577 74.087) (end 84.695 74.205) (width 0.254) (layer B.Cu) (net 24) (status 30))
 (segment (start 84.695 74.205) (end 84.323 74.577) (width 0.254) (layer F.Cu) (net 24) (status 30))
 (segment (start 101.341 74.651) (end 100.895 74.205) (width 0.254) (layer F.Cu) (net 24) (status 30))
 (segment (start 101.341 78.655) (end 101.341 74.651) (width 0.254) (layer F.Cu) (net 24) (status 20))
 (segment (start 100.071 79.925) (end 101.341 78.655) (width 0.254) (layer F.Cu) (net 24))
 (segment (start 85.593 79.925) (end 100.071 79.925) (width 0.254) (layer F.Cu) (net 24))
 (segment (start 84.323 78.655) (end 85.593 79.925) (width 0.254) (layer F.Cu) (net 24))
 (segment (start 84.323 74.577) (end 84.323 78.655) (width 0.254) (layer F.Cu) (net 24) (status 10))
 (segment (start 76.7538 66.6408) (end 76.2204 66.1074) (width 0.254) (layer B.Cu) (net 24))
 (segment (start 78.5318 66.6408) (end 76.7538 66.6408) (width 0.254) (layer B.Cu) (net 24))
 (segment (start 79.0906 67.1996) (end 78.5318 66.6408) (width 0.254) (layer B.Cu) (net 24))
 (segment (start 79.751 67.1996) (end 79.0906 67.1996) (width 0.254) (layer B.Cu) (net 24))
 (segment (start 84.732 72.1806) (end 79.751 67.1996) (width 0.254) (layer B.Cu) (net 24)))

